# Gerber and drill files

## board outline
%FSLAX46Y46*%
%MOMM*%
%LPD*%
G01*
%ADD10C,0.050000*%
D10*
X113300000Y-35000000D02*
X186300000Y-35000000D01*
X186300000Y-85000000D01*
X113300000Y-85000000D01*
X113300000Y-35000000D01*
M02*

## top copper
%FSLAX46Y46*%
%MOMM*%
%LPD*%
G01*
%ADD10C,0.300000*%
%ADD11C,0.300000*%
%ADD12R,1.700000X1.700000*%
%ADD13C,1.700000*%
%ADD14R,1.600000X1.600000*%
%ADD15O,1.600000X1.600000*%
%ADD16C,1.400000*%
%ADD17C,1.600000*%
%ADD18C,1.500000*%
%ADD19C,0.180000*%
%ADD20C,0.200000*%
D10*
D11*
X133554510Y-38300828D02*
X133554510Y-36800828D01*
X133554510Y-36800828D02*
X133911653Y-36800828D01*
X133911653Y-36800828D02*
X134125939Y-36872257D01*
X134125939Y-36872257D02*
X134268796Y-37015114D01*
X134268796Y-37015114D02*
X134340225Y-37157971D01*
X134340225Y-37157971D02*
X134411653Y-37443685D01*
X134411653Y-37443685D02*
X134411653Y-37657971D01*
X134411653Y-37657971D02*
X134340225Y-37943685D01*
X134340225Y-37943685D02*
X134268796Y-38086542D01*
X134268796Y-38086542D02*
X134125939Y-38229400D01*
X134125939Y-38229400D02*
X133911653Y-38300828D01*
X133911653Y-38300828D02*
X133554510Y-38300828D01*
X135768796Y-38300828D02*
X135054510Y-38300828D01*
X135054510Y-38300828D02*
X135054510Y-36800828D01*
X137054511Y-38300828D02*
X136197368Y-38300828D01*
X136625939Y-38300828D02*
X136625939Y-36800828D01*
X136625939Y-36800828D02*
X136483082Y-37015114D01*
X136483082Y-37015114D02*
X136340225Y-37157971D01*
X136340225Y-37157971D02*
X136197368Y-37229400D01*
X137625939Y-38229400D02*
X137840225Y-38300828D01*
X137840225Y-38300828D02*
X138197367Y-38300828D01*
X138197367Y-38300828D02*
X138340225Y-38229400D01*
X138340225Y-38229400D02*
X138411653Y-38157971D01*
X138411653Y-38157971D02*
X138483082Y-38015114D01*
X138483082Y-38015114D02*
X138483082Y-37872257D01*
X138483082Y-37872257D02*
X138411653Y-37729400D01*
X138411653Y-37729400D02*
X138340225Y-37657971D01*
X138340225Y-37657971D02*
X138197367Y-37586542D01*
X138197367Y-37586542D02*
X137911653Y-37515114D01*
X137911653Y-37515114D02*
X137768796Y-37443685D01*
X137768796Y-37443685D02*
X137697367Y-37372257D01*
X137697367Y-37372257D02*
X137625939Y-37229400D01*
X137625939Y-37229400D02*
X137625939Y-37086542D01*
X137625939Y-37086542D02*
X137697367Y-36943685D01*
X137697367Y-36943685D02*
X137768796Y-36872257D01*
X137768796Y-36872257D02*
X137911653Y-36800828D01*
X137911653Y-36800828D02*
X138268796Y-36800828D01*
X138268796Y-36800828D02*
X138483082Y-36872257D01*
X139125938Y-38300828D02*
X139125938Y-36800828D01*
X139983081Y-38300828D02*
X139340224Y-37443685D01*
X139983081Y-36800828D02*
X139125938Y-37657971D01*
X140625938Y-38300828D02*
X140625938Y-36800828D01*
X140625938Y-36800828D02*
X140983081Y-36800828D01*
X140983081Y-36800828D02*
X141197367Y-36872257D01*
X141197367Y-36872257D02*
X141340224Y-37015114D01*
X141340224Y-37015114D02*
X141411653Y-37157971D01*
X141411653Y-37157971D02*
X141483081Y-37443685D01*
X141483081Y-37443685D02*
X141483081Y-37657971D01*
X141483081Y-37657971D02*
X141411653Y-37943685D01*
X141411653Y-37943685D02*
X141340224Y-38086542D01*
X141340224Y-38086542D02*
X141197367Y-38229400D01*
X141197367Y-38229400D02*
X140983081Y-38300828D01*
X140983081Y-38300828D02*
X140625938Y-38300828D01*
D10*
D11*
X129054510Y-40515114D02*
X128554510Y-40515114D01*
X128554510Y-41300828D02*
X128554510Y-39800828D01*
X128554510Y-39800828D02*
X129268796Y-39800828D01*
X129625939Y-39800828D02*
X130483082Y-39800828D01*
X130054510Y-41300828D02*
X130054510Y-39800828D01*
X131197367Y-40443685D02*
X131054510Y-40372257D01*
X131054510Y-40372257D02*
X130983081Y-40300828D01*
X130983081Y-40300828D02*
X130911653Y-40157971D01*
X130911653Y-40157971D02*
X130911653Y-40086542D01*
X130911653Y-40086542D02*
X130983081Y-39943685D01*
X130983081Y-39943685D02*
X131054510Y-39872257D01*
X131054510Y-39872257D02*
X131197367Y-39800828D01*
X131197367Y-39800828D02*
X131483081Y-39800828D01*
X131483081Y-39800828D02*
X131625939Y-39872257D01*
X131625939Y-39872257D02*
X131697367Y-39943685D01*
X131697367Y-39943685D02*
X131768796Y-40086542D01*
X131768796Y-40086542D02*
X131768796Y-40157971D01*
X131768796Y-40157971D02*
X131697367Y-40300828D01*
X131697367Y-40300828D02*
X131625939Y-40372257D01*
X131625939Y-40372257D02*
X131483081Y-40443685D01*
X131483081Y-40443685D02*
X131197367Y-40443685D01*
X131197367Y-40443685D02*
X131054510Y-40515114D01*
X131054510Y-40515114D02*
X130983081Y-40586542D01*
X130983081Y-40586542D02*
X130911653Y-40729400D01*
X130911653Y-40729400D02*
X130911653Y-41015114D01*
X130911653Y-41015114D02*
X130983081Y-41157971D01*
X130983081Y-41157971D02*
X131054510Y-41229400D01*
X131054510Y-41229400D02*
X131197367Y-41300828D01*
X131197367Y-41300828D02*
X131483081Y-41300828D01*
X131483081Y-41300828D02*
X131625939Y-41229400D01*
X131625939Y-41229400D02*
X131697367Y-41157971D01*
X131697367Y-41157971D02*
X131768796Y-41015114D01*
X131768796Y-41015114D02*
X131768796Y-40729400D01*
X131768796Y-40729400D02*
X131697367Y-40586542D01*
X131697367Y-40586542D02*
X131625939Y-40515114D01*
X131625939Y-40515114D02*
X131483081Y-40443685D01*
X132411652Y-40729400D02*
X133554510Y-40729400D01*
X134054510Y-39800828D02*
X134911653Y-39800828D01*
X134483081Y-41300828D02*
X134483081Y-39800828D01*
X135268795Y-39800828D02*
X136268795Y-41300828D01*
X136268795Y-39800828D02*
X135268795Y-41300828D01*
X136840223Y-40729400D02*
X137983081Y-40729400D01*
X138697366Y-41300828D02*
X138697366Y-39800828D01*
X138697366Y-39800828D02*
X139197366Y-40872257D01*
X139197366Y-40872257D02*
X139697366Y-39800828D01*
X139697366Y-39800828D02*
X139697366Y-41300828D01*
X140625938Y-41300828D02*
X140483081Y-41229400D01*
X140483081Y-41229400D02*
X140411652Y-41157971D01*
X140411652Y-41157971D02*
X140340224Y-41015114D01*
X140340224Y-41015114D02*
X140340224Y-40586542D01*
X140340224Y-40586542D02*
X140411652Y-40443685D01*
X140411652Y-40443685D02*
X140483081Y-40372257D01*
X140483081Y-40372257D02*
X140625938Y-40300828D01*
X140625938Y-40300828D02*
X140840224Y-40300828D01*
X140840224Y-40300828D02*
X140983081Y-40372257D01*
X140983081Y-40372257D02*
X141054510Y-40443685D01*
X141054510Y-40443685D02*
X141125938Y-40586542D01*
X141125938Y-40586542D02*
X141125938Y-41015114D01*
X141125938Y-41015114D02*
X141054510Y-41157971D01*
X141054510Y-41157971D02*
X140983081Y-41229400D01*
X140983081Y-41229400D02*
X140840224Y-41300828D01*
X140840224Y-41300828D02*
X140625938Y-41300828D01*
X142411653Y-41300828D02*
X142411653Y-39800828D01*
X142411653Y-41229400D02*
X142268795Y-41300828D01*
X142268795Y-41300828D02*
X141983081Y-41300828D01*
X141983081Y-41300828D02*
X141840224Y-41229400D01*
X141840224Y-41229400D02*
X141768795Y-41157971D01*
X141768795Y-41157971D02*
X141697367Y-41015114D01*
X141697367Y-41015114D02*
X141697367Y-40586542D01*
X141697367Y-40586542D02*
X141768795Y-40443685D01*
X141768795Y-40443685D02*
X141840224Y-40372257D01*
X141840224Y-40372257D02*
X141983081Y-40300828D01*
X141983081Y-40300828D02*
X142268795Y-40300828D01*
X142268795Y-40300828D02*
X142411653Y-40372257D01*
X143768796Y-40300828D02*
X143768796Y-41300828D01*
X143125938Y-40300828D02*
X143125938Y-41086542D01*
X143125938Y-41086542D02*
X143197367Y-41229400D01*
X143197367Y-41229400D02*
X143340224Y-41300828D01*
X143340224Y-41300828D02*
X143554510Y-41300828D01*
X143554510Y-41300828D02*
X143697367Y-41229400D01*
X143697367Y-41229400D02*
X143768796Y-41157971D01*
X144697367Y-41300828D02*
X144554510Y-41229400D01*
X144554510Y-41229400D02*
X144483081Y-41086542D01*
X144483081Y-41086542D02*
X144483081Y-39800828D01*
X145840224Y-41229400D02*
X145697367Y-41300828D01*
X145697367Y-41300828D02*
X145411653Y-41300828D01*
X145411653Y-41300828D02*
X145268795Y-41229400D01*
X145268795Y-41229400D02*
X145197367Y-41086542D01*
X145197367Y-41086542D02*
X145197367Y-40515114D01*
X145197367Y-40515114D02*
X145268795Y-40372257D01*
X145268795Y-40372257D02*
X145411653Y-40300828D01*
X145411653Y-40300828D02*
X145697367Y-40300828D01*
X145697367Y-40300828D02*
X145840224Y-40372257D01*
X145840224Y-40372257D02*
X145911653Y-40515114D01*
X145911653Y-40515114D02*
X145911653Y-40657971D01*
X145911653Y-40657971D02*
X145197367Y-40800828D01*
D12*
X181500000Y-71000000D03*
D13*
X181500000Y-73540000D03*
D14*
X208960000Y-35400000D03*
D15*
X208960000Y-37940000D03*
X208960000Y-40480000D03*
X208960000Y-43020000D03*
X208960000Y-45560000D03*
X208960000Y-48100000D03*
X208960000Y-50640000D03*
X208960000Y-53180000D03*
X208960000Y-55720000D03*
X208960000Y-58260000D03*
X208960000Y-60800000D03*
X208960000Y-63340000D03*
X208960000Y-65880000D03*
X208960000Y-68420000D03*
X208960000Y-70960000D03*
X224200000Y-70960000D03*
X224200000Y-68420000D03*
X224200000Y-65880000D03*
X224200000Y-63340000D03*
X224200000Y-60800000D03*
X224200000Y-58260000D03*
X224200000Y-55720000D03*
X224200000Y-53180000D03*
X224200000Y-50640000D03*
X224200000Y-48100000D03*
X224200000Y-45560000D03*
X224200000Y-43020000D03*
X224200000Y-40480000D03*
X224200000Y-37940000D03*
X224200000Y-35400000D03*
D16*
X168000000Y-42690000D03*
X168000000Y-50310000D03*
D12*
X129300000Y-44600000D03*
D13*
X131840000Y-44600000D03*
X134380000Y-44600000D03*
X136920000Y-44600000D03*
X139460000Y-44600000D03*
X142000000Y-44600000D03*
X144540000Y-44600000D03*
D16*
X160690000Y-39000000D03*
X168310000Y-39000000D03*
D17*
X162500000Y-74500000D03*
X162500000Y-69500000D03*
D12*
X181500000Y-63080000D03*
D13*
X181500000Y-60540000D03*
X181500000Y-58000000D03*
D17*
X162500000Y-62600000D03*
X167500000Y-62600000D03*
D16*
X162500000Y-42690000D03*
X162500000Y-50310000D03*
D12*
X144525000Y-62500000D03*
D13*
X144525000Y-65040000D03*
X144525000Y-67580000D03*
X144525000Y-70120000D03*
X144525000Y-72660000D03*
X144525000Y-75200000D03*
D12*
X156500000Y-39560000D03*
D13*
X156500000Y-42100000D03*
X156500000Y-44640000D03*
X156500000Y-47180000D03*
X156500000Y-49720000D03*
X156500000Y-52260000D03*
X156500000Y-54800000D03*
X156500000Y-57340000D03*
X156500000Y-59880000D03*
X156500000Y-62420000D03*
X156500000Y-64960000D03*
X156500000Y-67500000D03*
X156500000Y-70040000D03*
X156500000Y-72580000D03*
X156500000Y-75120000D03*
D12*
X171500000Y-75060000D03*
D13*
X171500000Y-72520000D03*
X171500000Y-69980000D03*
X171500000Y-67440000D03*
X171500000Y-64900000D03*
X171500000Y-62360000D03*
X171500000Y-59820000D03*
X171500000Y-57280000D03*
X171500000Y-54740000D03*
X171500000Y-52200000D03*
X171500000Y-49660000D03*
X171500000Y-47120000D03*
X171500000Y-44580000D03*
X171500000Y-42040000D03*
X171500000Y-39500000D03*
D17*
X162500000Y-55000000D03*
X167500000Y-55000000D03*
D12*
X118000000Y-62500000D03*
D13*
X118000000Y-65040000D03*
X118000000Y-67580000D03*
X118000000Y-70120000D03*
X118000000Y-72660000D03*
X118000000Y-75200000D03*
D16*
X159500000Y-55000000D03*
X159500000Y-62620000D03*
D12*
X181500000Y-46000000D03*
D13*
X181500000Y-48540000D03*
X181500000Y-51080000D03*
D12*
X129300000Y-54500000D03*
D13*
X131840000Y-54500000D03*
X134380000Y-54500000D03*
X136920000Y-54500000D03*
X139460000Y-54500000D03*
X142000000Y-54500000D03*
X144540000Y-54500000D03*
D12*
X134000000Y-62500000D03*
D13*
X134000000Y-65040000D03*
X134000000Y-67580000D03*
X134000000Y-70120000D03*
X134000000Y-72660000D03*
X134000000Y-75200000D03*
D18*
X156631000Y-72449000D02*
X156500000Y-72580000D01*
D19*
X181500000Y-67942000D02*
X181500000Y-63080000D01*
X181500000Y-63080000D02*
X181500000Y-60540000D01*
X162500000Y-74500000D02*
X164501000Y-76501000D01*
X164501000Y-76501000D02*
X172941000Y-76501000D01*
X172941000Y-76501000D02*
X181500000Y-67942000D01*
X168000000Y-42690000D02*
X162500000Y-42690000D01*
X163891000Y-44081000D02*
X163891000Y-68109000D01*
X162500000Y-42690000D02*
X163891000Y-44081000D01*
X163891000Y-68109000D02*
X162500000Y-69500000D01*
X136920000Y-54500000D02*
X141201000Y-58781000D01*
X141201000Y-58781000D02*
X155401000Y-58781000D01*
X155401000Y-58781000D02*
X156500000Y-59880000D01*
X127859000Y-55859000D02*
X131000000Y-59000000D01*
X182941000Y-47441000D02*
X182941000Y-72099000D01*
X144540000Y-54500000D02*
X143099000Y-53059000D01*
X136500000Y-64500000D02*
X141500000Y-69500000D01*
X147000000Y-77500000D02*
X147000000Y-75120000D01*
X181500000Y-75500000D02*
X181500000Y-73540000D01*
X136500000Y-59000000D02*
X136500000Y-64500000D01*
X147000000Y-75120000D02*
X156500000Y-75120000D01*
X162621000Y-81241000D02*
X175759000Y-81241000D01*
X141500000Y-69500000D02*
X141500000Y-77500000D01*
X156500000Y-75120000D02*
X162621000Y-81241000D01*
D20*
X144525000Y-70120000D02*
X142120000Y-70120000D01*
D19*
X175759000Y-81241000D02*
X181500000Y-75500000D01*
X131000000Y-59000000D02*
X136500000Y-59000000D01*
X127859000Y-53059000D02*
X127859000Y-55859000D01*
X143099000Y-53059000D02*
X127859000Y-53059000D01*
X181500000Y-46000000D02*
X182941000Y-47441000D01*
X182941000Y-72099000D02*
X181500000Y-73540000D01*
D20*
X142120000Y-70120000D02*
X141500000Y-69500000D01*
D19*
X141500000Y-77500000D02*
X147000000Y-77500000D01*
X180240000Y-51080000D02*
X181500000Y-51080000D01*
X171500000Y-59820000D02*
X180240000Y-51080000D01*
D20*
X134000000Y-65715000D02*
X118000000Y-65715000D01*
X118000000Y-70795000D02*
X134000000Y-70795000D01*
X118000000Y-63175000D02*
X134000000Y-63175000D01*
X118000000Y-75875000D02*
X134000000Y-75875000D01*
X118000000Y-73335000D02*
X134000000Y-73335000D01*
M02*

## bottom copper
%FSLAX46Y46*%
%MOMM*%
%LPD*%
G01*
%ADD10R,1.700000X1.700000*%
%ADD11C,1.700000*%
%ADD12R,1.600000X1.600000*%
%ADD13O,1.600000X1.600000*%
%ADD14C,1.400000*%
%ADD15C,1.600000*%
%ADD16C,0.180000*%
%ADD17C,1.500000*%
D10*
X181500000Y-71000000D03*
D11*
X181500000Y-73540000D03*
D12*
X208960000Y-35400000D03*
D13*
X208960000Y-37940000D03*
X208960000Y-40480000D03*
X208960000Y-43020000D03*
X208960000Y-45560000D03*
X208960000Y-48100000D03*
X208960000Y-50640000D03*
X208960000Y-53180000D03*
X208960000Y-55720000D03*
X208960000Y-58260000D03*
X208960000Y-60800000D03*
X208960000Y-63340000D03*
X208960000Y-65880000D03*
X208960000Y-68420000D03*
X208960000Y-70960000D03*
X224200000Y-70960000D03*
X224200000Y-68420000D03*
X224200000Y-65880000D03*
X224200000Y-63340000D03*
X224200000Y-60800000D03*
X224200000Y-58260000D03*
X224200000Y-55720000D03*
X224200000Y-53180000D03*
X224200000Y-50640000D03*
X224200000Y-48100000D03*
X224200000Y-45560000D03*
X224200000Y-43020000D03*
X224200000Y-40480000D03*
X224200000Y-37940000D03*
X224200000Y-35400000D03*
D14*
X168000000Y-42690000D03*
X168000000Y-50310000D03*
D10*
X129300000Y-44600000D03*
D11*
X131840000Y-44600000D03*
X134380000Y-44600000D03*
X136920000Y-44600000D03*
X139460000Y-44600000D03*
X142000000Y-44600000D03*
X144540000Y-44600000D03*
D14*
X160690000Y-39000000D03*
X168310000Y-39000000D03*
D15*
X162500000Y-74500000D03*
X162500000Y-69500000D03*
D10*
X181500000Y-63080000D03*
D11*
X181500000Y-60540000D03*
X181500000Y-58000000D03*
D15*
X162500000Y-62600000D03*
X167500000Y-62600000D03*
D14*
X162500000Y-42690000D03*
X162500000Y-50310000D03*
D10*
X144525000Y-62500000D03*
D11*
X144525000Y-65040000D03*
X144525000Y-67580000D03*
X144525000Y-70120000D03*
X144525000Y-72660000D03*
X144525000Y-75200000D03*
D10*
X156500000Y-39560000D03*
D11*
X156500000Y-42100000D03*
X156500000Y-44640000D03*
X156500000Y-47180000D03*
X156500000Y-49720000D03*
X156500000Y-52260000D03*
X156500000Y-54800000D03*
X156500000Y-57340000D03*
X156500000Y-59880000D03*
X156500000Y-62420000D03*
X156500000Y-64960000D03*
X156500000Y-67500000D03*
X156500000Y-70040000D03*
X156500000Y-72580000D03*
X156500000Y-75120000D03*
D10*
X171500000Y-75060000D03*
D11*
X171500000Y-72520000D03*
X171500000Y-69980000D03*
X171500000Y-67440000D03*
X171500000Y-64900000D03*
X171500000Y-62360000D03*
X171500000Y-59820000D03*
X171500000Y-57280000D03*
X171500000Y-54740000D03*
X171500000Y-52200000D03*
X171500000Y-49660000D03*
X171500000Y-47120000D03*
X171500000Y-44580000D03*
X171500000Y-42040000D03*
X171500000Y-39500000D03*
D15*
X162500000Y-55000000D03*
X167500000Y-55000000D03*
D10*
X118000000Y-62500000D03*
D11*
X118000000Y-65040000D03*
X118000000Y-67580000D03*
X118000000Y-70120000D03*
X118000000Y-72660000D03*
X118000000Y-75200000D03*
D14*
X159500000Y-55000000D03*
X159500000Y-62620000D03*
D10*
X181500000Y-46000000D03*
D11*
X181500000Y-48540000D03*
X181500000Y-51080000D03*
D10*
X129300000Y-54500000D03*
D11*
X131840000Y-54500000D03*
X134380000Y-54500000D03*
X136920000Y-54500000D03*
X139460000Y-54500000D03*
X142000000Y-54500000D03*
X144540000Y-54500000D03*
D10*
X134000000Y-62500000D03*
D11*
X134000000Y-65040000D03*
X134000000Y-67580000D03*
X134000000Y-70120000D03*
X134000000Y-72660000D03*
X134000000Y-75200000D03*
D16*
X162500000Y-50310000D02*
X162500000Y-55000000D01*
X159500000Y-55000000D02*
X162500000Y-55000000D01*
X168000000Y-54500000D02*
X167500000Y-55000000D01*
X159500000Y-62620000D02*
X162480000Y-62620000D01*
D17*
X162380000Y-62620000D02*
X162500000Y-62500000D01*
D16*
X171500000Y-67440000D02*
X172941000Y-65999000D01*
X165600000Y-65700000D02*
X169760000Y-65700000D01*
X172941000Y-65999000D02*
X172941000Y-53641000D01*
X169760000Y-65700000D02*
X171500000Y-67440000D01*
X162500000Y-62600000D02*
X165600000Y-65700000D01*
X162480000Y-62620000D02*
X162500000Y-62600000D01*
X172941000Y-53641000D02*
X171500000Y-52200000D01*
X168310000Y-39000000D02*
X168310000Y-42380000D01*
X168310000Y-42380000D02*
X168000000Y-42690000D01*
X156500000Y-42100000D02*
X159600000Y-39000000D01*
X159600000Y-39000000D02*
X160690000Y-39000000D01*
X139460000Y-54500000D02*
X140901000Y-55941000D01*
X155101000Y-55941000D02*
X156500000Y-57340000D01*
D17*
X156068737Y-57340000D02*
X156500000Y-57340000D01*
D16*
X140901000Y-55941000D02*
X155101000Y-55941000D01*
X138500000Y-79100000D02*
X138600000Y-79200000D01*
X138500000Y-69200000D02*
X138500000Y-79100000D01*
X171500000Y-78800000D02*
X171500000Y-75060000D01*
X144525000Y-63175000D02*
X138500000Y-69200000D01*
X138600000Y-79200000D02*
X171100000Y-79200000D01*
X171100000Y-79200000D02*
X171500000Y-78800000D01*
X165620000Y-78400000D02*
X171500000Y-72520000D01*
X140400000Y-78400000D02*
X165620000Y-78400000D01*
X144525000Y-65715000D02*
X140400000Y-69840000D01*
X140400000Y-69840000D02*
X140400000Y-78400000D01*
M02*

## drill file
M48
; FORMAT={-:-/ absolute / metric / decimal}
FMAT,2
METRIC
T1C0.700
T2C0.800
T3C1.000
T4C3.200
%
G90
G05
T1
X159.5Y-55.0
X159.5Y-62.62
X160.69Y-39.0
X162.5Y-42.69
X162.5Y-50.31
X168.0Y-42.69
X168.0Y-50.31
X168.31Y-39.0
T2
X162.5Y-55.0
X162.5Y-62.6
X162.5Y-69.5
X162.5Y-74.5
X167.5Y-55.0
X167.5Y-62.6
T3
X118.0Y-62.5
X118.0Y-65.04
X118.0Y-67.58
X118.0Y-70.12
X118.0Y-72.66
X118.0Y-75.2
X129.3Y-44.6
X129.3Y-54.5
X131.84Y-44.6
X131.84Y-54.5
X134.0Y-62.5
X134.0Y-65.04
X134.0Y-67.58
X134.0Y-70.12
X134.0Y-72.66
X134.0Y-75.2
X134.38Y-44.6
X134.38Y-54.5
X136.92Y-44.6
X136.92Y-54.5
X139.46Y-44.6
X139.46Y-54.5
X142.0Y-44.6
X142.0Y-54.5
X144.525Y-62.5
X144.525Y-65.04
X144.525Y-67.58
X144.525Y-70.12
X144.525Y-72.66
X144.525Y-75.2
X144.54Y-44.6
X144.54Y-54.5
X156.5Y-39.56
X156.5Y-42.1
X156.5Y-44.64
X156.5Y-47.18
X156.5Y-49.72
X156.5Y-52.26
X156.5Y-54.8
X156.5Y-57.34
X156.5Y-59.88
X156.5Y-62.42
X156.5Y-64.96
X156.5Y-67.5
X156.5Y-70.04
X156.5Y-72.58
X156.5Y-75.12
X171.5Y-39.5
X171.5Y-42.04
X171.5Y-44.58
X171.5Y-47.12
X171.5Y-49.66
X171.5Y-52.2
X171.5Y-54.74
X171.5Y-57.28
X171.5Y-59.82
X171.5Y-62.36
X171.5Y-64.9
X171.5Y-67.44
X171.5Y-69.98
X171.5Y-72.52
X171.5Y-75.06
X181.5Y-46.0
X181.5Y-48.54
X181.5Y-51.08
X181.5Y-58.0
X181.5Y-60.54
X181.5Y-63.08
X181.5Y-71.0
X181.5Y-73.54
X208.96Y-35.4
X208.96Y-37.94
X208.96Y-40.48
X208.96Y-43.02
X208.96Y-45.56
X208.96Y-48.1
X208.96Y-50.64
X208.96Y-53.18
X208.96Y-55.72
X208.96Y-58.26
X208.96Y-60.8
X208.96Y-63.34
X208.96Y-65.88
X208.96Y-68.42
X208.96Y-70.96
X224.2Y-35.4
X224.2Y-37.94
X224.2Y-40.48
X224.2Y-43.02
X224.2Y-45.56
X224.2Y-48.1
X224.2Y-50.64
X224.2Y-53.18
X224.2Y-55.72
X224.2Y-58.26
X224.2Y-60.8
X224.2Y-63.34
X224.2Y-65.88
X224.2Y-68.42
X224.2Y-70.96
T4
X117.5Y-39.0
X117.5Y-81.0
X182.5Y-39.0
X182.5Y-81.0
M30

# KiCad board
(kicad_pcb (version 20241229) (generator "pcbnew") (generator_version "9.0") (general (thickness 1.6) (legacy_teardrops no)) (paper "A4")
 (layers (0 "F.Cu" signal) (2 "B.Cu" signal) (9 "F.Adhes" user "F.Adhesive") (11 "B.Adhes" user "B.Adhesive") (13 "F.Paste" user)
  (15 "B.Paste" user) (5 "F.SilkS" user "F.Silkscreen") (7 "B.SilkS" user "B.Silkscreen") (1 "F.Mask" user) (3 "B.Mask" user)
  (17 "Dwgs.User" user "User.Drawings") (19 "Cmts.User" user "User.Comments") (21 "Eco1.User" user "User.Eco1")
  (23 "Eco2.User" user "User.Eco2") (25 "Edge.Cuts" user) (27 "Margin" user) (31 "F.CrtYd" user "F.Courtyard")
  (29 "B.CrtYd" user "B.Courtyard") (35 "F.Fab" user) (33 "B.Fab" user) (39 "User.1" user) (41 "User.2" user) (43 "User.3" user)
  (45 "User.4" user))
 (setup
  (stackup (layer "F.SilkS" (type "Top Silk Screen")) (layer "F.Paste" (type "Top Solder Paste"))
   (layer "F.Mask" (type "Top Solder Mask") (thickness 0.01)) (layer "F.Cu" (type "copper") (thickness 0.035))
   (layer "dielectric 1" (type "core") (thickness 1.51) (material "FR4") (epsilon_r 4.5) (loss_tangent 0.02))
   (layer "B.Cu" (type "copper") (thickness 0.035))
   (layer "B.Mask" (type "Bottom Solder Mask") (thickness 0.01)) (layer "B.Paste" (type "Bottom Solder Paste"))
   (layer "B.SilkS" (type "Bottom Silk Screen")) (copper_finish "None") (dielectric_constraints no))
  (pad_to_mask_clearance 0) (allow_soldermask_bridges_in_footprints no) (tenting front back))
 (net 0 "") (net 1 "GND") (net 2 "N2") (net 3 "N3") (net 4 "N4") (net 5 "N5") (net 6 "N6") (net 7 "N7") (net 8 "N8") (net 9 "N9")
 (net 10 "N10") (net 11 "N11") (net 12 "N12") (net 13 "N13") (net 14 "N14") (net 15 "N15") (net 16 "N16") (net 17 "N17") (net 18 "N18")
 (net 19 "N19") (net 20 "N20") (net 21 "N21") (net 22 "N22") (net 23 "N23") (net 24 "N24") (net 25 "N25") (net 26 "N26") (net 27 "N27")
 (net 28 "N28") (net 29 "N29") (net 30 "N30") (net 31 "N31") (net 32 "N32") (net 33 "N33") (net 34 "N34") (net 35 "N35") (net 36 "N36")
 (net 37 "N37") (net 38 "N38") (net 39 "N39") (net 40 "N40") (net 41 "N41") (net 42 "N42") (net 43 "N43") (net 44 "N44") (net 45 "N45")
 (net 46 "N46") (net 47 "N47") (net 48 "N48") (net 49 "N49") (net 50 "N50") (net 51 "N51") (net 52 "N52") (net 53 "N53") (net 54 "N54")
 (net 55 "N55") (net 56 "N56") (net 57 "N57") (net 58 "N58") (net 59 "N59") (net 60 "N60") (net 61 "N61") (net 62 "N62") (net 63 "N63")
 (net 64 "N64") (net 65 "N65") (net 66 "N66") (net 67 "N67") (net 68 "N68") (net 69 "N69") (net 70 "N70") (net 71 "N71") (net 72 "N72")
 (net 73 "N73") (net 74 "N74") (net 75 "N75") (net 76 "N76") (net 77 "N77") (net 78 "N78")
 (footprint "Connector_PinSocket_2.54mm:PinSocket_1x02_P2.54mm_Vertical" (layer "F.Cu") (at 181.5 71)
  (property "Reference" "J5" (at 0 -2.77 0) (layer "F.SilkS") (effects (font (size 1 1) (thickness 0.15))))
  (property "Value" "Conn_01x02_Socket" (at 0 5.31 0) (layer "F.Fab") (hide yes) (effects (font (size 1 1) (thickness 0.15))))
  (pad "1" thru_hole rect (at 0 0) (size 1.7 1.7) (drill 1) (layers "*.Cu" "*.Mask") (remove_unused_layers no) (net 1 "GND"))
  (pad "2" thru_hole circle (at 0 2.54) (size 1.7 1.7) (drill 1) (layers "*.Cu" "*.Mask") (remove_unused_layers no) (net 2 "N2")))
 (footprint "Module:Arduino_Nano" (layer "F.Cu") (at 208.96 35.4)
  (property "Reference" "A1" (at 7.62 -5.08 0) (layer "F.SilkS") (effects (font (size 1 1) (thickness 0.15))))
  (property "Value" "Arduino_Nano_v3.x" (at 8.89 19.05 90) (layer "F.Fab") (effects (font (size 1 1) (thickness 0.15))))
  (pad "1" thru_hole rect (at 0 0) (size 1.6 1.6) (drill 1) (layers "*.Cu" "*.Mask") (remove_unused_layers no) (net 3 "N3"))
  (pad "2" thru_hole oval (at 0 2.54) (size 1.6 1.6) (drill 1) (layers "*.Cu" "*.Mask") (remove_unused_layers no) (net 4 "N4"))
  (pad "3" thru_hole oval (at 0 5.08) (size 1.6 1.6) (drill 1) (layers "*.Cu" "*.Mask") (remove_unused_layers no) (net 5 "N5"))
  (pad "4" thru_hole oval (at 0 7.62) (size 1.6 1.6) (drill 1) (layers "*.Cu" "*.Mask") (remove_unused_layers no) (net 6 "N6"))
  (pad "5" thru_hole oval (at 0 10.16) (size 1.6 1.6) (drill 1) (layers "*.Cu" "*.Mask") (remove_unused_layers no) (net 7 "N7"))
  (pad "6" thru_hole oval (at 0 12.7) (size 1.6 1.6) (drill 1) (layers "*.Cu" "*.Mask") (remove_unused_layers no) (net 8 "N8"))
  (pad "7" thru_hole oval (at 0 15.24) (size 1.6 1.6) (drill 1) (layers "*.Cu" "*.Mask") (remove_unused_layers no) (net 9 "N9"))
  (pad "8" thru_hole oval (at 0 17.78) (size 1.6 1.6) (drill 1) (layers "*.Cu" "*.Mask") (remove_unused_layers no) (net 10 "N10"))
  (pad "9" thru_hole oval (at 0 20.32) (size 1.6 1.6) (drill 1) (layers "*.Cu" "*.Mask") (remove_unused_layers no) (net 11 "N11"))
  (pad "10" thru_hole oval (at 0 22.86) (size 1.6 1.6) (drill 1) (layers "*.Cu" "*.Mask") (remove_unused_layers no) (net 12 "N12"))
  (pad "11" thru_hole oval (at 0 25.4) (size 1.6 1.6) (drill 1) (layers "*.Cu" "*.Mask") (remove_unused_layers no) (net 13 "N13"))
  (pad "12" thru_hole oval (at 0 27.94) (size 1.6 1.6) (drill 1) (layers "*.Cu" "*.Mask") (remove_unused_layers no) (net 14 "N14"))
  (pad "13" thru_hole oval (at 0 30.48) (size 1.6 1.6) (drill 1) (layers "*.Cu" "*.Mask") (remove_unused_layers no) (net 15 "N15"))
  (pad "14" thru_hole oval (at 0 33.02) (size 1.6 1.6) (drill 1) (layers "*.Cu" "*.Mask") (remove_unused_layers no) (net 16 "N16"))
  (pad "15" thru_hole oval (at 0 35.56) (size 1.6 1.6) (drill 1) (layers "*.Cu" "*.Mask") (remove_unused_layers no) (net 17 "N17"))
  (pad "16" thru_hole oval (at 15.24 35.56) (size 1.6 1.6) (drill 1) (layers "*.Cu" "*.Mask") (remove_unused_layers no) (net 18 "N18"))
  (pad "17" thru_hole oval (at 15.24 33.02) (size 1.6 1.6) (drill 1) (layers "*.Cu" "*.Mask") (remove_unused_layers no) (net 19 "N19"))
  (pad "18" thru_hole oval (at 15.24 30.48) (size 1.6 1.6) (drill 1) (layers "*.Cu" "*.Mask") (remove_unused_layers no) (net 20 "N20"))
  (pad "19" thru_hole oval (at 15.24 27.94) (size 1.6 1.6) (drill 1) (layers "*.Cu" "*.Mask") (remove_unused_layers no) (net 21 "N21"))
  (pad "20" thru_hole oval (at 15.24 25.4) (size 1.6 1.6) (drill 1) (layers "*.Cu" "*.Mask") (remove_unused_layers no) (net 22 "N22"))
  (pad "21" thru_hole oval (at 15.24 22.86) (size 1.6 1.6) (drill 1) (layers "*.Cu" "*.Mask") (remove_unused_layers no) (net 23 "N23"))
  (pad "22" thru_hole oval (at 15.24 20.32) (size 1.6 1.6) (drill 1) (layers "*.Cu" "*.Mask") (remove_unused_layers no) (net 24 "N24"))
  (pad "23" thru_hole oval (at 15.24 17.78) (size 1.6 1.6) (drill 1) (layers "*.Cu" "*.Mask") (remove_unused_layers no) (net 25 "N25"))
  (pad "24" thru_hole oval (at 15.24 15.24) (size 1.6 1.6) (drill 1) (layers "*.Cu" "*.Mask") (remove_unused_layers no) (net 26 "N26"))
  (pad "25" thru_hole oval (at 15.24 12.7) (size 1.6 1.6) (drill 1) (layers "*.Cu" "*.Mask") (remove_unused_layers no) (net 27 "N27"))
  (pad "26" thru_hole oval (at 15.24 10.16) (size 1.6 1.6) (drill 1) (layers "*.Cu" "*.Mask") (remove_unused_layers no) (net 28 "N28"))
  (pad "27" thru_hole oval (at 15.24 7.62) (size 1.6 1.6) (drill 1) (layers "*.Cu" "*.Mask") (remove_unused_layers no) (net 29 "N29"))
  (pad "28" thru_hole oval (at 15.24 5.08) (size 1.6 1.6) (drill 1) (layers "*.Cu" "*.Mask") (remove_unused_layers no) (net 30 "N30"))
  (pad "29" thru_hole oval (at 15.24 2.54) (size 1.6 1.6) (drill 1) (layers "*.Cu" "*.Mask") (remove_unused_layers no) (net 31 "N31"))
  (pad "30" thru_hole oval (at 15.24 0) (size 1.6 1.6) (drill 1) (layers "*.Cu" "*.Mask") (remove_unused_layers no) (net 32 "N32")))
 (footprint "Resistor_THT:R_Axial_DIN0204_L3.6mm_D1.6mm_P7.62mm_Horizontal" (layer "F.Cu") (at 168 42.69 -90)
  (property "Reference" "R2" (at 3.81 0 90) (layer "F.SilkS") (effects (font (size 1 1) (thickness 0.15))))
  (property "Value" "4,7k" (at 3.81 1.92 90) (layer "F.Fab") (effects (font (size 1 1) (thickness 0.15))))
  (pad "1" thru_hole circle (at 0 0 270) (size 1.4 1.4) (drill 0.7) (layers "*.Cu" "*.Mask") (remove_unused_layers no) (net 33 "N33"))
  (pad "2" thru_hole circle (at 7.62 0 270) (size 1.4 1.4) (drill 0.7) (layers "*.Cu" "*.Mask") (remove_unused_layers no) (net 1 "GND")))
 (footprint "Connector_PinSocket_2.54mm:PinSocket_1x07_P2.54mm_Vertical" (layer "F.Cu") (at 129.3 44.6 90)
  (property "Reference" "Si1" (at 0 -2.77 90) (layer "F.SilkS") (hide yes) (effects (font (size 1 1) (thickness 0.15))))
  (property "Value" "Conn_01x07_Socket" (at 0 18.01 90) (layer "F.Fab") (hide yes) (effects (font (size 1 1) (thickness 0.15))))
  (pad "1" thru_hole rect (at 0 0 90) (size 1.7 1.7) (drill 1) (layers "*.Cu" "*.Mask") (remove_unused_layers no) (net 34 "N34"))
  (pad "2" thru_hole circle (at 0 2.54 90) (size 1.7 1.7) (drill 1) (layers "*.Cu" "*.Mask") (remove_unused_layers no) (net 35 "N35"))
  (pad "3" thru_hole circle (at 0 5.08 90) (size 1.7 1.7) (drill 1) (layers "*.Cu" "*.Mask") (remove_unused_layers no) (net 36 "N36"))
  (pad "4" thru_hole circle (at 0 7.62 90) (size 1.7 1.7) (drill 1) (layers "*.Cu" "*.Mask") (remove_unused_layers no) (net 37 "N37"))
  (pad "5" thru_hole circle (at 0 10.16 90) (size 1.7 1.7) (drill 1) (layers "*.Cu" "*.Mask") (remove_unused_layers no) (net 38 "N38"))
  (pad "6" thru_hole circle (at 0 12.7 90) (size 1.7 1.7) (drill 1) (layers "*.Cu" "*.Mask") (remove_unused_layers no) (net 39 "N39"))
  (pad "7" thru_hole circle (at 0 15.24 90) (size 1.7 1.7) (drill 1) (layers "*.Cu" "*.Mask") (remove_unused_layers no) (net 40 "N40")))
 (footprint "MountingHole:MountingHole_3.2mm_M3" (layer "F.Cu") (at 182.5 81)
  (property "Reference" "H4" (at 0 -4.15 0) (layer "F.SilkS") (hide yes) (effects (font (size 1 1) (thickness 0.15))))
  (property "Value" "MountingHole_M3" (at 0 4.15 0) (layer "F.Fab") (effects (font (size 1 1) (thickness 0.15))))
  (pad "" np_thru_hole circle (at 0 0) (size 3.2 3.2) (drill 3.2) (layers "*.Cu" "*.Mask")))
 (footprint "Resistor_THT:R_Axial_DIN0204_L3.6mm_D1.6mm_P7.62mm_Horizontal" (layer "F.Cu") (at 160.69 39)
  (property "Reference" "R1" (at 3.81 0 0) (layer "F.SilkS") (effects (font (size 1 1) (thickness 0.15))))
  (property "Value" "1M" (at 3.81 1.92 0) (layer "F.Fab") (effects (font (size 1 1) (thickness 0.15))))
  (pad "1" thru_hole circle (at 0 0) (size 1.4 1.4) (drill 0.7) (layers "*.Cu" "*.Mask") (remove_unused_layers no) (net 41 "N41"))
  (pad "2" thru_hole circle (at 7.62 0) (size 1.4 1.4) (drill 0.7) (layers "*.Cu" "*.Mask") (remove_unused_layers no) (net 33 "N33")))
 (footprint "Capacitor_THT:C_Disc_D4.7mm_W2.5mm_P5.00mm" (layer "F.Cu") (at 162.5 74.5 90)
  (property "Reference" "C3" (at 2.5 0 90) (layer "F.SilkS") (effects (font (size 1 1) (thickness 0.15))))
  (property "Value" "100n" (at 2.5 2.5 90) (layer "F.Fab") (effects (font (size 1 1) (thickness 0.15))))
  (pad "1" thru_hole circle (at 0 0 90) (size 1.6 1.6) (drill 0.8) (layers "*.Cu" "*.Mask") (remove_unused_layers no) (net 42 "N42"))
  (pad "2" thru_hole circle (at 5 0 90) (size 1.6 1.6) (drill 0.8) (layers "*.Cu" "*.Mask") (remove_unused_layers no) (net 33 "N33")))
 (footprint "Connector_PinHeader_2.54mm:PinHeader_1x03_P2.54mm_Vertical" (layer "F.Cu") (at 181.5 63.08 180)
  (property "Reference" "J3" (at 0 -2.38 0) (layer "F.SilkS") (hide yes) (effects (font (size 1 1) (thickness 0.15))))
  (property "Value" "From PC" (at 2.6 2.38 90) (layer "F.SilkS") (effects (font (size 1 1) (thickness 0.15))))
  (pad "1" thru_hole rect (at 0 0 180) (size 1.7 1.7) (drill 1) (layers "*.Cu" "*.Mask") (remove_unused_layers no) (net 42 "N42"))
  (pad "2" thru_hole circle (at 0 2.54 180) (size 1.7 1.7) (drill 1) (layers "*.Cu" "*.Mask") (remove_unused_layers no) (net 42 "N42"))
  (pad "3" thru_hole circle (at 0 5.08 180) (size 1.7 1.7) (drill 1) (layers "*.Cu" "*.Mask") (remove_unused_layers no) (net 1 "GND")))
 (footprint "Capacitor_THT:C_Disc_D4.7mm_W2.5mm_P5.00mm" (layer "F.Cu") (at 162.5 62.6)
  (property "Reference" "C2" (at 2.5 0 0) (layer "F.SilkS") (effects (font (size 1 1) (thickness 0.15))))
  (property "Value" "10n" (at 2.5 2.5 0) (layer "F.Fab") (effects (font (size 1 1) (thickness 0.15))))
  (pad "1" thru_hole circle (at 0 0) (size 1.6 1.6) (drill 0.8) (layers "*.Cu" "*.Mask") (remove_unused_layers no) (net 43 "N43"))
  (pad "2" thru_hole circle (at 5 0) (size 1.6 1.6) (drill 0.8) (layers "*.Cu" "*.Mask") (remove_unused_layers no) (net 1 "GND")))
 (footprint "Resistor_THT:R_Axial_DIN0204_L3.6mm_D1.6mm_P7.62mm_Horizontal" (layer "F.Cu") (at 162.5 42.69 -90)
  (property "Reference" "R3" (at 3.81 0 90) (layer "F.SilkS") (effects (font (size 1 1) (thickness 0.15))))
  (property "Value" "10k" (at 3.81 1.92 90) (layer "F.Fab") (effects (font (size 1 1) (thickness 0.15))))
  (pad "1" thru_hole circle (at 0 0 270) (size 1.4 1.4) (drill 0.7) (layers "*.Cu" "*.Mask") (remove_unused_layers no) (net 33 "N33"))
  (pad "2" thru_hole circle (at 7.62 0 270) (size 1.4 1.4) (drill 0.7) (layers "*.Cu" "*.Mask") (remove_unused_layers no) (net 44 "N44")))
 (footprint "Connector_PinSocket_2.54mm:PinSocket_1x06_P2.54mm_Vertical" (layer "F.Cu") (at 144.525 62.5)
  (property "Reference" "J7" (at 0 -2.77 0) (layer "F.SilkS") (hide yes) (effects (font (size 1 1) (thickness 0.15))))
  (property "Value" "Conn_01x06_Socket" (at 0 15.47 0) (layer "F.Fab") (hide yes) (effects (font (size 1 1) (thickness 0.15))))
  (pad "1" thru_hole rect (at 0 0) (size 1.7 1.7) (drill 1) (layers "*.Cu" "*.Mask") (remove_unused_layers no) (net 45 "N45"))
  (pad "2" thru_hole circle (at 0 2.54) (size 1.7 1.7) (drill 1) (layers "*.Cu" "*.Mask") (remove_unused_layers no) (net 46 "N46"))
  (pad "3" thru_hole circle (at 0 5.08) (size 1.7 1.7) (drill 1) (layers "*.Cu" "*.Mask") (remove_unused_layers no) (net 1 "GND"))
  (pad "4" thru_hole circle (at 0 7.62) (size 1.7 1.7) (drill 1) (layers "*.Cu" "*.Mask") (remove_unused_layers no) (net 2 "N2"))
  (pad "5" thru_hole circle (at 0 10.16) (size 1.7 1.7) (drill 1) (layers "*.Cu" "*.Mask") (remove_unused_layers no) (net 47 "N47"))
  (pad "6" thru_hole circle (at 0 12.7) (size 1.7 1.7) (drill 1) (layers "*.Cu" "*.Mask") (remove_unused_layers no) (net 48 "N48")))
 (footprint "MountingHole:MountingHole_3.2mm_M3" (layer "F.Cu") (at 117.5 39)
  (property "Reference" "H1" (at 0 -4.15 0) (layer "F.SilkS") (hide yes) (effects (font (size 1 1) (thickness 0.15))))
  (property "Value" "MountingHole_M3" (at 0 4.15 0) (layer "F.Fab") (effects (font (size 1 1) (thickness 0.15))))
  (pad "" np_thru_hole circle (at 0 0) (size 3.2 3.2) (drill 3.2) (layers "*.Cu" "*.Mask")))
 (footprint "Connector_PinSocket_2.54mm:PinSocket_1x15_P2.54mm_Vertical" (layer "F.Cu") (at 156.5 39.56)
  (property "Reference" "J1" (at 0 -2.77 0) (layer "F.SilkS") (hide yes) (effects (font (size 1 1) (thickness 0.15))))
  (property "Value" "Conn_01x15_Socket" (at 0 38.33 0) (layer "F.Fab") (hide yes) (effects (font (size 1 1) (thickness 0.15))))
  (pad "1" thru_hole rect (at 0 0) (size 1.7 1.7) (drill 1) (layers "*.Cu" "*.Mask") (remove_unused_layers no) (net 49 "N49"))
  (pad "2" thru_hole circle (at 0 2.54) (size 1.7 1.7) (drill 1) (layers "*.Cu" "*.Mask") (remove_unused_layers no) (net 41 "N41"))
  (pad "3" thru_hole circle (at 0 5.08) (size 1.7 1.7) (drill 1) (layers "*.Cu" "*.Mask") (remove_unused_layers no) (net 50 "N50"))
  (pad "4" thru_hole circle (at 0 7.62) (size 1.7 1.7) (drill 1) (layers "*.Cu" "*.Mask") (remove_unused_layers no) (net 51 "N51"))
  (pad "5" thru_hole circle (at 0 10.16) (size 1.7 1.7) (drill 1) (layers "*.Cu" "*.Mask") (remove_unused_layers no) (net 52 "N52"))
  (pad "6" thru_hole circle (at 0 12.7) (size 1.7 1.7) (drill 1) (layers "*.Cu" "*.Mask") (remove_unused_layers no) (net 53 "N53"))
  (pad "7" thru_hole circle (at 0 15.24) (size 1.7 1.7) (drill 1) (layers "*.Cu" "*.Mask") (remove_unused_layers no) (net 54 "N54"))
  (pad "8" thru_hole circle (at 0 17.78) (size 1.7 1.7) (drill 1) (layers "*.Cu" "*.Mask") (remove_unused_layers no) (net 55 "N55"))
  (pad "9" thru_hole circle (at 0 20.32) (size 1.7 1.7) (drill 1) (layers "*.Cu" "*.Mask") (remove_unused_layers no) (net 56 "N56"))
  (pad "10" thru_hole circle (at 0 22.86) (size 1.7 1.7) (drill 1) (layers "*.Cu" "*.Mask") (remove_unused_layers no) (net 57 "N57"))
  (pad "11" thru_hole circle (at 0 25.4) (size 1.7 1.7) (drill 1) (layers "*.Cu" "*.Mask") (remove_unused_layers no) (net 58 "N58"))
  (pad "12" thru_hole circle (at 0 27.94) (size 1.7 1.7) (drill 1) (layers "*.Cu" "*.Mask") (remove_unused_layers no) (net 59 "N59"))
  (pad "13" thru_hole circle (at 0 30.48) (size 1.7 1.7) (drill 1) (layers "*.Cu" "*.Mask") (remove_unused_layers no) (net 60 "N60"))
  (pad "14" thru_hole circle (at 0 33.02) (size 1.7 1.7) (drill 1) (layers "*.Cu" "*.Mask") (remove_unused_layers no) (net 1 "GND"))
  (pad "15" thru_hole circle (at 0 35.56) (size 1.7 1.7) (drill 1) (layers "*.Cu" "*.Mask") (remove_unused_layers no) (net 2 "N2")))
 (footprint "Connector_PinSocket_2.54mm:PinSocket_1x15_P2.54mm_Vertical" (layer "F.Cu") (at 171.5 75.06 180)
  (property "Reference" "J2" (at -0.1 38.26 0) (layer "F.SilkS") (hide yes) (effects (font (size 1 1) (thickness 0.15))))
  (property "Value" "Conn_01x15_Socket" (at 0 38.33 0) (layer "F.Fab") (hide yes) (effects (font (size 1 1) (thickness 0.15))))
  (pad "1" thru_hole rect (at 0 0 180) (size 1.7 1.7) (drill 1) (layers "*.Cu" "*.Mask") (remove_unused_layers no) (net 45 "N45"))
  (pad "2" thru_hole circle (at 0 2.54 180) (size 1.7 1.7) (drill 1) (layers "*.Cu" "*.Mask") (remove_unused_layers no) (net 46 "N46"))
  (pad "3" thru_hole circle (at 0 5.08 180) (size 1.7 1.7) (drill 1) (layers "*.Cu" "*.Mask") (remove_unused_layers no) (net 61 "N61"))
  (pad "4" thru_hole circle (at 0 7.62 180) (size 1.7 1.7) (drill 1) (layers "*.Cu" "*.Mask") (remove_unused_layers no) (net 43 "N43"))
  (pad "5" thru_hole circle (at 0 10.16 180) (size 1.7 1.7) (drill 1) (layers "*.Cu" "*.Mask") (remove_unused_layers no) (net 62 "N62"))
  (pad "6" thru_hole circle (at 0 12.7 180) (size 1.7 1.7) (drill 1) (layers "*.Cu" "*.Mask") (remove_unused_layers no) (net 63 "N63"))
  (pad "7" thru_hole circle (at 0 15.24 180) (size 1.7 1.7) (drill 1) (layers "*.Cu" "*.Mask") (remove_unused_layers no) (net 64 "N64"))
  (pad "8" thru_hole circle (at 0 17.78 180) (size 1.7 1.7) (drill 1) (layers "*.Cu" "*.Mask") (remove_unused_layers no) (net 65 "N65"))
  (pad "9" thru_hole circle (at 0 20.32 180) (size 1.7 1.7) (drill 1) (layers "*.Cu" "*.Mask") (remove_unused_layers no) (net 1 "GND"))
  (pad "10" thru_hole circle (at 0 22.86 180) (size 1.7 1.7) (drill 1) (layers "*.Cu" "*.Mask") (remove_unused_layers no) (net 43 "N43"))
  (pad "11" thru_hole circle (at 0 25.4 180) (size 1.7 1.7) (drill 1) (layers "*.Cu" "*.Mask") (remove_unused_layers no) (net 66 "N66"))
  (pad "12" thru_hole circle (at 0 27.94 180) (size 1.7 1.7) (drill 1) (layers "*.Cu" "*.Mask") (remove_unused_layers no) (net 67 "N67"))
  (pad "13" thru_hole circle (at 0 30.48 180) (size 1.7 1.7) (drill 1) (layers "*.Cu" "*.Mask") (remove_unused_layers no) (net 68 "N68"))
  (pad "14" thru_hole circle (at 0 33.02 180) (size 1.7 1.7) (drill 1) (layers "*.Cu" "*.Mask") (remove_unused_layers no) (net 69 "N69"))
  (pad "15" thru_hole circle (at 0 35.56 180) (size 1.7 1.7) (drill 1) (layers "*.Cu" "*.Mask") (remove_unused_layers no) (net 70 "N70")))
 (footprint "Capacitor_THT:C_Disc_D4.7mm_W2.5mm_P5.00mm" (layer "F.Cu") (at 162.5 55)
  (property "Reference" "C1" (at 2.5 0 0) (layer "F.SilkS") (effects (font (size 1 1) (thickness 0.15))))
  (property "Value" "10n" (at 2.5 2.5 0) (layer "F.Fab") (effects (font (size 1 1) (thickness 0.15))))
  (pad "1" thru_hole circle (at 0 0) (size 1.6 1.6) (drill 0.8) (layers "*.Cu" "*.Mask") (remove_unused_layers no) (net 44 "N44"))
  (pad "2" thru_hole circle (at 5 0) (size 1.6 1.6) (drill 0.8) (layers "*.Cu" "*.Mask") (remove_unused_layers no) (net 1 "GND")))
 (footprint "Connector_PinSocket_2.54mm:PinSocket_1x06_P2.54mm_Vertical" (layer "F.Cu") (at 118 62.5)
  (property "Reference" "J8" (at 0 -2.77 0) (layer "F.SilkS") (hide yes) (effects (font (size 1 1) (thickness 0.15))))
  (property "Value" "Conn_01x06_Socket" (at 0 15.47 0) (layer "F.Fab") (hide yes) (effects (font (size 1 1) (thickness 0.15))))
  (pad "1" thru_hole rect (at 0 0) (size 1.7 1.7) (drill 1) (layers "*.Cu" "*.Mask") (remove_unused_layers no) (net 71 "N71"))
  (pad "2" thru_hole circle (at 0 2.54) (size 1.7 1.7) (drill 1) (layers "*.Cu" "*.Mask") (remove_unused_layers no) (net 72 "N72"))
  (pad "3" thru_hole circle (at 0 5.08) (size 1.7 1.7) (drill 1) (layers "*.Cu" "*.Mask") (remove_unused_layers no) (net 1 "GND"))
  (pad "4" thru_hole circle (at 0 7.62) (size 1.7 1.7) (drill 1) (layers "*.Cu" "*.Mask") (remove_unused_layers no) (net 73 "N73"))
  (pad "5" thru_hole circle (at 0 10.16) (size 1.7 1.7) (drill 1) (layers "*.Cu" "*.Mask") (remove_unused_layers no) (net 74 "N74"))
  (pad "6" thru_hole circle (at 0 12.7) (size 1.7 1.7) (drill 1) (layers "*.Cu" "*.Mask") (remove_unused_layers no) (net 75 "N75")))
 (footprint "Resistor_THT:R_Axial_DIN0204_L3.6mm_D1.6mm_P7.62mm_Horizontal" (layer "F.Cu") (at 159.5 55 -90)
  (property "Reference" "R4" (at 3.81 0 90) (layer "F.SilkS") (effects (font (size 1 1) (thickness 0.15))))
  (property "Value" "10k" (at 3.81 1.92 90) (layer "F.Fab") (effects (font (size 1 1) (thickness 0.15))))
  (pad "1" thru_hole circle (at 0 0 270) (size 1.4 1.4) (drill 0.7) (layers "*.Cu" "*.Mask") (remove_unused_layers no) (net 44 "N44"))
  (pad "2" thru_hole circle (at 7.62 0 270) (size 1.4 1.4) (drill 0.7) (layers "*.Cu" "*.Mask") (remove_unused_layers no) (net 43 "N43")))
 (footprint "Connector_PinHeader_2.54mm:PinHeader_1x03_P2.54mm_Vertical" (layer "F.Cu") (at 181.5 46)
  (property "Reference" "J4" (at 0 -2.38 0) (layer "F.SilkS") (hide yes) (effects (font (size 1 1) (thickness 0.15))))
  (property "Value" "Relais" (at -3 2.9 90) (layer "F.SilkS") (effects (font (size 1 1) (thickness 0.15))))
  (pad "1" thru_hole rect (at 0 0) (size 1.7 1.7) (drill 1) (layers "*.Cu" "*.Mask") (remove_unused_layers no) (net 2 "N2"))
  (pad "2" thru_hole circle (at 0 2.54) (size 1.7 1.7) (drill 1) (layers "*.Cu" "*.Mask") (remove_unused_layers no) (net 1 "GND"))
  (pad "3" thru_hole circle (at 0 5.08) (size 1.7 1.7) (drill 1) (layers "*.Cu" "*.Mask") (remove_unused_layers no) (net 64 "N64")))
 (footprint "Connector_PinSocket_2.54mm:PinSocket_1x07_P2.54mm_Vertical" (layer "F.Cu") (at 129.3 54.5 90)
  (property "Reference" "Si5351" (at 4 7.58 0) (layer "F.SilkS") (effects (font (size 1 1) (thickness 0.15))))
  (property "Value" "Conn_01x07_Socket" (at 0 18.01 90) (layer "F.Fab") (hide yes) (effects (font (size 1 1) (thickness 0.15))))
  (pad "1" thru_hole rect (at 0 0 90) (size 1.7 1.7) (drill 1) (layers "*.Cu" "*.Mask") (remove_unused_layers no) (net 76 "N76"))
  (pad "2" thru_hole circle (at 0 2.54 90) (size 1.7 1.7) (drill 1) (layers "*.Cu" "*.Mask") (remove_unused_layers no) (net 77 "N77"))
  (pad "3" thru_hole circle (at 0 5.08 90) (size 1.7 1.7) (drill 1) (layers "*.Cu" "*.Mask") (remove_unused_layers no) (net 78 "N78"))
  (pad "4" thru_hole circle (at 0 7.62 90) (size 1.7 1.7) (drill 1) (layers "*.Cu" "*.Mask") (remove_unused_layers no) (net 56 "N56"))
  (pad "5" thru_hole circle (at 0 10.16 90) (size 1.7 1.7) (drill 1) (layers "*.Cu" "*.Mask") (remove_unused_layers no) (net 55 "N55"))
  (pad "6" thru_hole circle (at 0 12.7 90) (size 1.7 1.7) (drill 1) (layers "*.Cu" "*.Mask") (remove_unused_layers no) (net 1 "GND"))
  (pad "7" thru_hole circle (at 0 15.24 90) (size 1.7 1.7) (drill 1) (layers "*.Cu" "*.Mask") (remove_unused_layers no) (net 2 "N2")))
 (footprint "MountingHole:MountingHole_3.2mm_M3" (layer "F.Cu") (at 117.5 81)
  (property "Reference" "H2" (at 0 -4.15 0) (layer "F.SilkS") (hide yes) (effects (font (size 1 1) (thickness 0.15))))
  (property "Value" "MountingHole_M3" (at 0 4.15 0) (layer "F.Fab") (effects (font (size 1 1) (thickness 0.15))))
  (pad "" np_thru_hole circle (at 0 0) (size 3.2 3.2) (drill 3.2) (layers "*.Cu" "*.Mask")))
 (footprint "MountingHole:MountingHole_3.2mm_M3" (layer "F.Cu") (at 182.5 39)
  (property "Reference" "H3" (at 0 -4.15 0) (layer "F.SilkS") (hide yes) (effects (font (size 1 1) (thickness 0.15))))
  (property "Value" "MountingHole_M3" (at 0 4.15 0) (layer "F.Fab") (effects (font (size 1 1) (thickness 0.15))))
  (pad "" np_thru_hole circle (at 0 0) (size 3.2 3.2) (drill 3.2) (layers "*.Cu" "*.Mask")))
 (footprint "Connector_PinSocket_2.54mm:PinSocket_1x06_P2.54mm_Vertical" (layer "F.Cu") (at 134 62.5)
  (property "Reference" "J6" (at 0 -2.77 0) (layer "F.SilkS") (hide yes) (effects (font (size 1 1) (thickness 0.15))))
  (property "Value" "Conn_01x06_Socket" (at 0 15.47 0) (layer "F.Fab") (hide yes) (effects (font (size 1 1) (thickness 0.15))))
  (pad "1" thru_hole rect (at 0 0) (size 1.7 1.7) (drill 1) (layers "*.Cu" "*.Mask") (remove_unused_layers no) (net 71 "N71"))
  (pad "2" thru_hole circle (at 0 2.54) (size 1.7 1.7) (drill 1) (layers "*.Cu" "*.Mask") (remove_unused_layers no) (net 72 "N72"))
  (pad "3" thru_hole circle (at 0 5.08) (size 1.7 1.7) (drill 1) (layers "*.Cu" "*.Mask") (remove_unused_layers no) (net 1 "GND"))
  (pad "4" thru_hole circle (at 0 7.62) (size 1.7 1.7) (drill 1) (layers "*.Cu" "*.Mask") (remove_unused_layers no) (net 73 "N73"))
  (pad "5" thru_hole circle (at 0 10.16) (size 1.7 1.7) (drill 1) (layers "*.Cu" "*.Mask") (remove_unused_layers no) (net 74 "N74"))
  (pad "6" thru_hole circle (at 0 12.7) (size 1.7 1.7) (drill 1) (layers "*.Cu" "*.Mask") (remove_unused_layers no) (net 75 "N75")))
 (gr_rect (start 113.3 35) (end 186.3 85) (stroke (width 0.05) (type default)) (fill no) (layer "Edge.Cuts"))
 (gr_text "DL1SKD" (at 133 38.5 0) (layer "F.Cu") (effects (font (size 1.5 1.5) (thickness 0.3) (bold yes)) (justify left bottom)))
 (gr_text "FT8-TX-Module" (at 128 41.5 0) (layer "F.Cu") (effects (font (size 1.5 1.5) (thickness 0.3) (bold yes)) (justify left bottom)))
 (segment (start 162.5 50.31) (end 162.5 55) (width 0.18) (layer "B.Cu") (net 44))
 (segment (start 159.5 55) (end 162.5 55) (width 0.18) (layer "B.Cu") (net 44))
 (segment (start 156.631 72.449) (end 156.5 72.58) (width 1.5) (layer "F.Cu") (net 1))
 (segment (start 168 54.5) (end 167.5 55) (width 0.18) (layer "B.Cu") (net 1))
 (segment (start 159.5 62.62) (end 162.48 62.62) (width 0.18) (layer "B.Cu") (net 43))
 (segment (start 162.38 62.62) (end 162.5 62.5) (width 1.5) (layer "B.Cu") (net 43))
 (segment (start 171.5 67.44) (end 172.941 65.999) (width 0.18) (layer "B.Cu") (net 43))
 (segment (start 165.6 65.7) (end 169.76 65.7) (width 0.18) (layer "B.Cu") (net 43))
 (segment (start 172.941 65.999) (end 172.941 53.641) (width 0.18) (layer "B.Cu") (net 43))
 (segment (start 169.76 65.7) (end 171.5 67.44) (width 0.18) (layer "B.Cu") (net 43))
 (segment (start 162.5 62.6) (end 165.6 65.7) (width 0.18) (layer "B.Cu") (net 43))
 (segment (start 162.48 62.62) (end 162.5 62.6) (width 0.18) (layer "B.Cu") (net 43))
 (segment (start 172.941 53.641) (end 171.5 52.2) (width 0.18) (layer "B.Cu") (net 43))
 (segment (start 181.5 67.942) (end 181.5 63.08) (width 0.18) (layer "F.Cu") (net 42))
 (segment (start 181.5 63.08) (end 181.5 60.54) (width 0.18) (layer "F.Cu") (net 42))
 (segment (start 162.5 74.5) (end 164.501 76.501) (width 0.18) (layer "F.Cu") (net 42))
 (segment (start 164.501 76.501) (end 172.941 76.501) (width 0.18) (layer "F.Cu") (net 42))
 (segment (start 172.941 76.501) (end 181.5 67.942) (width 0.18) (layer "F.Cu") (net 42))
 (segment (start 168 42.69) (end 162.5 42.69) (width 0.18) (layer "F.Cu") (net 33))
 (segment (start 163.891 44.081) (end 163.891 68.109) (width 0.18) (layer "F.Cu") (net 33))
 (segment (start 162.5 42.69) (end 163.891 44.081) (width 0.18) (layer "F.Cu") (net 33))
 (segment (start 163.891 68.109) (end 162.5 69.5) (width 0.18) (layer "F.Cu") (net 33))
 (segment (start 168.31 39) (end 168.31 42.38) (width 0.18) (layer "B.Cu") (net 33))
 (segment (start 168.31 42.38) (end 168 42.69) (width 0.18) (layer "B.Cu") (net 33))
 (segment (start 136.92 54.5) (end 141.201 58.781) (width 0.18) (layer "F.Cu") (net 56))
 (segment (start 141.201 58.781) (end 155.401 58.781) (width 0.18) (layer "F.Cu") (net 56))
 (segment (start 155.401 58.781) (end 156.5 59.88) (width 0.18) (layer "F.Cu") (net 56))
 (segment (start 156.5 42.1) (end 159.6 39) (width 0.18) (layer "B.Cu") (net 41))
 (segment (start 159.6 39) (end 160.69 39) (width 0.18) (layer "B.Cu") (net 41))
 (segment (start 127.859 55.859) (end 131 59) (width 0.18) (layer "F.Cu") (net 2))
 (segment (start 182.941 47.441) (end 182.941 72.099) (width 0.18) (layer "F.Cu") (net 2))
 (segment (start 144.54 54.5) (end 143.099 53.059) (width 0.18) (layer "F.Cu") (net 2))
 (segment (start 136.5 64.5) (end 141.5 69.5) (width 0.18) (layer "F.Cu") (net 2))
 (segment (start 147 77.5) (end 147 75.12) (width 0.18) (layer "F.Cu") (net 2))
 (segment (start 181.5 75.5) (end 181.5 73.54) (width 0.18) (layer "F.Cu") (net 2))
 (segment (start 136.5 59) (end 136.5 64.5) (width 0.18) (layer "F.Cu") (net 2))
 (segment (start 147 75.12) (end 156.5 75.12) (width 0.18) (layer "F.Cu") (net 2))
 (segment (start 162.621 81.241) (end 175.759 81.241) (width 0.18) (layer "F.Cu") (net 2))
 (segment (start 141.5 69.5) (end 141.5 77.5) (width 0.18) (layer "F.Cu") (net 2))
 (segment (start 156.5 75.12) (end 162.621 81.241) (width 0.18) (layer "F.Cu") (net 2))
 (segment (start 144.525 70.12) (end 142.12 70.12) (width 0.2) (layer "F.Cu") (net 2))
 (segment (start 175.759 81.241) (end 181.5 75.5) (width 0.18) (layer "F.Cu") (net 2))
 (segment (start 131 59) (end 136.5 59) (width 0.18) (layer "F.Cu") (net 2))
 (segment (start 127.859 53.059) (end 127.859 55.859) (width 0.18) (layer "F.Cu") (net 2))
 (segment (start 143.099 53.059) (end 127.859 53.059) (width 0.18) (layer "F.Cu") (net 2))
 (segment (start 181.5 46) (end 182.941 47.441) (width 0.18) (layer "F.Cu") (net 2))
 (segment (start 182.941 72.099) (end 181.5 73.54) (width 0.18) (layer "F.Cu") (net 2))
 (segment (start 142.12 70.12) (end 141.5 69.5) (width 0.2) (layer "F.Cu") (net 2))
 (segment (start 141.5 77.5) (end 147 77.5) (width 0.18) (layer "F.Cu") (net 2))
 (segment (start 139.46 54.5) (end 140.901 55.941) (width 0.18) (layer "B.Cu") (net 55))
 (segment (start 155.101 55.941) (end 156.5 57.34) (width 0.18) (layer "B.Cu") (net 55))
 (segment (start 156.068737 57.34) (end 156.5 57.34) (width 1.5) (layer "B.Cu") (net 55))
 (segment (start 140.901 55.941) (end 155.101 55.941) (width 0.18) (layer "B.Cu") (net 55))
 (segment (start 138.5 79.1) (end 138.6 79.2) (width 0.18) (layer "B.Cu") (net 45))
 (segment (start 138.5 69.2) (end 138.5 79.1) (width 0.18) (layer "B.Cu") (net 45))
 (segment (start 171.5 78.8) (end 171.5 75.06) (width 0.18) (layer "B.Cu") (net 45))
 (segment (start 144.525 63.175) (end 138.5 69.2) (width 0.18) (layer "B.Cu") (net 45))
 (segment (start 138.6 79.2) (end 171.1 79.2) (width 0.18) (layer "B.Cu") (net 45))
 (segment (start 171.1 79.2) (end 171.5 78.8) (width 0.18) (layer "B.Cu") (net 45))
 (segment (start 165.62 78.4) (end 171.5 72.52) (width 0.18) (layer "B.Cu") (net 46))
 (segment (start 140.4 78.4) (end 165.62 78.4) (width 0.18) (layer "B.Cu") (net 46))
 (segment (start 144.525 65.715) (end 140.4 69.84) (width 0.18) (layer "B.Cu") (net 46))
 (segment (start 140.4 69.84) (end 140.4 78.4) (width 0.18) (layer "B.Cu") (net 46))
 (segment (start 180.24 51.08) (end 181.5 51.08) (width 0.18) (layer "F.Cu") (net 64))
 (segment (start 171.5 59.82) (end 180.24 51.08) (width 0.18) (layer "F.Cu") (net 64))
 (segment (start 134 65.715) (end 118 65.715) (width 0.2) (layer "F.Cu") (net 72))
 (segment (start 118 70.795) (end 134 70.795) (width 0.2) (layer "F.Cu") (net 73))
 (segment (start 118 63.175) (end 134 63.175) (width 0.2) (layer "F.Cu") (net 71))
 (segment (start 118 75.875) (end 134 75.875) (width 0.2) (layer "F.Cu") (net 75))
 (segment (start 118 73.335) (end 134 73.335) (width 0.2) (layer "F.Cu") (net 74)))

